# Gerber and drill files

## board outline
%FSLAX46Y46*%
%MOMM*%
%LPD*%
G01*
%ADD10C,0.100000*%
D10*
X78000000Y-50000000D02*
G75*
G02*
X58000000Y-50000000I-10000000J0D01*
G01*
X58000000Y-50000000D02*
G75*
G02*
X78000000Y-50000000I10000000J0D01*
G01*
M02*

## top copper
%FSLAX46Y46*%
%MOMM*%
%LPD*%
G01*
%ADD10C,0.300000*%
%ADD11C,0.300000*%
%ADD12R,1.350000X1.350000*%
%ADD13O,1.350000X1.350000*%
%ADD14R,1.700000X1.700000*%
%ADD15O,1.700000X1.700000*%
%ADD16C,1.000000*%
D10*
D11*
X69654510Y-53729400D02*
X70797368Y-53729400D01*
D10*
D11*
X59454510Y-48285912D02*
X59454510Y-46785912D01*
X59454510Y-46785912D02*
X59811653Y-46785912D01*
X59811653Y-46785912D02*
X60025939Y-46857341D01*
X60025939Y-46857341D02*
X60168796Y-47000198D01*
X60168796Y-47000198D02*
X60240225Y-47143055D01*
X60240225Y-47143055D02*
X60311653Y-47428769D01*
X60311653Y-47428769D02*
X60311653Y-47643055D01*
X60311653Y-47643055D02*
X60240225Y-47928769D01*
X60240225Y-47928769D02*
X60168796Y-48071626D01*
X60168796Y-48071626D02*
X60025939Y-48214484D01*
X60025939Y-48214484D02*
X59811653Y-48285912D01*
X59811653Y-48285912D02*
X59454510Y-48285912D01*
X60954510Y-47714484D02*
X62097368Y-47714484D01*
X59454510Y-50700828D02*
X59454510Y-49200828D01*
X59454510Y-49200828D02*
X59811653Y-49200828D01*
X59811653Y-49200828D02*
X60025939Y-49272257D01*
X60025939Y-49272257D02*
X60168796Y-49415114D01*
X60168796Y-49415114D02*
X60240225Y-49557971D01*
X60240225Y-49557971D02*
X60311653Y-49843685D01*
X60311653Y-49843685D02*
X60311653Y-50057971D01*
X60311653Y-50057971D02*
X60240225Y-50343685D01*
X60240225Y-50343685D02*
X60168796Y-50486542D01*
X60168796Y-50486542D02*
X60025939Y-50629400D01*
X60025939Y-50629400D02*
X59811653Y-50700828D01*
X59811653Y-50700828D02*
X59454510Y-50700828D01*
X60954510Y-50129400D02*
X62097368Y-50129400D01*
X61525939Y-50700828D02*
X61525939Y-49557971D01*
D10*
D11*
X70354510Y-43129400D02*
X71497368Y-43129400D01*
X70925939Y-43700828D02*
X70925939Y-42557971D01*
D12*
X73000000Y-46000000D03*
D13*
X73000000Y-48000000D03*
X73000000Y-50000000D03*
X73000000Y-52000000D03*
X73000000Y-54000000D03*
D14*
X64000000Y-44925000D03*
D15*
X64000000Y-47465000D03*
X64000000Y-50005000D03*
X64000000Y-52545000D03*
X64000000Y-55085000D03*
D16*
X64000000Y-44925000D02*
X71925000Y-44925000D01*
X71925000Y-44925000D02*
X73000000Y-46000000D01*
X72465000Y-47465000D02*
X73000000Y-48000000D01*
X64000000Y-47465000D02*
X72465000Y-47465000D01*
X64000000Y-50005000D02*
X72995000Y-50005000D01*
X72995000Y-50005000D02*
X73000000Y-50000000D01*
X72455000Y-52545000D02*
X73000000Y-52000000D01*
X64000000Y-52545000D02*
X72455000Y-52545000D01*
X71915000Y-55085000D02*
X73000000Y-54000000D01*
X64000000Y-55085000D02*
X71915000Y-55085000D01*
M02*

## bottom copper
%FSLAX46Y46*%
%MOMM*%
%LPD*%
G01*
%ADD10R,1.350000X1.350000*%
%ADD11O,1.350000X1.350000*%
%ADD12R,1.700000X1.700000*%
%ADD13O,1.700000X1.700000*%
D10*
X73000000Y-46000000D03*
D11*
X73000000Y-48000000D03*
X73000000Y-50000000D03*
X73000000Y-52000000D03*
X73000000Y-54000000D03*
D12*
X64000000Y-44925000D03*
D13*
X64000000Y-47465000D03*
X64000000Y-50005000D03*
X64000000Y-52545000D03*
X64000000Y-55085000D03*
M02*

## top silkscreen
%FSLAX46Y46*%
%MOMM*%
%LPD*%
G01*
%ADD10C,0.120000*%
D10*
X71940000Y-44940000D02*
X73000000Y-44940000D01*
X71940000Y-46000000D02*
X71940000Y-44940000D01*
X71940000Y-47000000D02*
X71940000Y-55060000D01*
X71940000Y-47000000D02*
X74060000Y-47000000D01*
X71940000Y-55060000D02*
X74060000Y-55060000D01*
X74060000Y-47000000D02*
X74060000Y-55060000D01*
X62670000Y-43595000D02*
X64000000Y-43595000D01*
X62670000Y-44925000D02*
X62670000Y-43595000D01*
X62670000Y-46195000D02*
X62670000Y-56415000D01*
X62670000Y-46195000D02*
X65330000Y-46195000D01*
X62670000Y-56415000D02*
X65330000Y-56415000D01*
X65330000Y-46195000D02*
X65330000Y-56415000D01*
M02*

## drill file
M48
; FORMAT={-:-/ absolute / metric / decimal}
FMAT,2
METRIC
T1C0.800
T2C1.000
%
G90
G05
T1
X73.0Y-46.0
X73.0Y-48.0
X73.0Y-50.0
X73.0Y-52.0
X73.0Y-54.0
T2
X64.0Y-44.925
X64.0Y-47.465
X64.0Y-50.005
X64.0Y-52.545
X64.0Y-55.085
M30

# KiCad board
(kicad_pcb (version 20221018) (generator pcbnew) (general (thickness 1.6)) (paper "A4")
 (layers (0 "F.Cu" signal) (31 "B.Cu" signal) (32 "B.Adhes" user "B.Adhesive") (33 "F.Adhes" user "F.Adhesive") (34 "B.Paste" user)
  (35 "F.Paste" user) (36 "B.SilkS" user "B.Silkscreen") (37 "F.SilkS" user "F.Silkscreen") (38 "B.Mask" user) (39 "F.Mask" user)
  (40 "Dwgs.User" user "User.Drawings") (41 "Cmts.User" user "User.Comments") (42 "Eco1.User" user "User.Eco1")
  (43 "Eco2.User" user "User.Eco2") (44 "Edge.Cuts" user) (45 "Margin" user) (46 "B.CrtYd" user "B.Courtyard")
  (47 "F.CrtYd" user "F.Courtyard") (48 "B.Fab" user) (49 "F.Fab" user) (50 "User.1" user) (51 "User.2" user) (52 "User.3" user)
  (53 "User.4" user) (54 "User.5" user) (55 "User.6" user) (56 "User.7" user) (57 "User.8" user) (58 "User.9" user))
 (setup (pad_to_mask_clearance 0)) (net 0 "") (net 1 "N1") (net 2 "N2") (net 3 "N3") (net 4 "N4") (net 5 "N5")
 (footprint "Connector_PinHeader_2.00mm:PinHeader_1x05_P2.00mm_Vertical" (layer "F.Cu") (at 73 46)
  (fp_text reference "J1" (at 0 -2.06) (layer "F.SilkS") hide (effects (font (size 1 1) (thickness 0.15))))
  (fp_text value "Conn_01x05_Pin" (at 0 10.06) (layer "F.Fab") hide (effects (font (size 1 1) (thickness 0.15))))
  (fp_line (start -1.06 -1.06) (end 0 -1.06) (stroke (width 0.12) (type solid)) (layer "F.SilkS"))
  (fp_line (start -1.06 0) (end -1.06 -1.06) (stroke (width 0.12) (type solid)) (layer "F.SilkS"))
  (fp_line (start -1.06 1) (end -1.06 9.06) (stroke (width 0.12) (type solid)) (layer "F.SilkS"))
  (fp_line (start -1.06 1) (end 1.06 1) (stroke (width 0.12) (type solid)) (layer "F.SilkS"))
  (fp_line (start -1.06 9.06) (end 1.06 9.06) (stroke (width 0.12) (type solid)) (layer "F.SilkS"))
  (fp_line (start 1.06 1) (end 1.06 9.06) (stroke (width 0.12) (type solid)) (layer "F.SilkS"))
  (pad "1" thru_hole rect (at 0 0) (size 1.35 1.35) (drill 0.8) (layers "*.Cu" "*.Mask") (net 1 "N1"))
  (pad "2" thru_hole oval (at 0 2) (size 1.35 1.35) (drill 0.8) (layers "*.Cu" "*.Mask") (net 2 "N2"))
  (pad "3" thru_hole oval (at 0 4) (size 1.35 1.35) (drill 0.8) (layers "*.Cu" "*.Mask") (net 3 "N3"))
  (pad "4" thru_hole oval (at 0 6) (size 1.35 1.35) (drill 0.8) (layers "*.Cu" "*.Mask") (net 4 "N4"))
  (pad "5" thru_hole oval (at 0 8) (size 1.35 1.35) (drill 0.8) (layers "*.Cu" "*.Mask") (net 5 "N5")))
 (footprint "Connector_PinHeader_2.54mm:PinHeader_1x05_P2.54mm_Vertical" (layer "F.Cu") (at 64 44.925)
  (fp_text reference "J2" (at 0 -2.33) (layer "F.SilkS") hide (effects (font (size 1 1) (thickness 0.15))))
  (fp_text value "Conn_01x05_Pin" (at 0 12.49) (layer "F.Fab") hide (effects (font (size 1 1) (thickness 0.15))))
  (fp_line (start -1.33 -1.33) (end 0 -1.33) (stroke (width 0.12) (type solid)) (layer "F.SilkS"))
  (fp_line (start -1.33 0) (end -1.33 -1.33) (stroke (width 0.12) (type solid)) (layer "F.SilkS"))
  (fp_line (start -1.33 1.27) (end -1.33 11.49) (stroke (width 0.12) (type solid)) (layer "F.SilkS"))
  (fp_line (start -1.33 1.27) (end 1.33 1.27) (stroke (width 0.12) (type solid)) (layer "F.SilkS"))
  (fp_line (start -1.33 11.49) (end 1.33 11.49) (stroke (width 0.12) (type solid)) (layer "F.SilkS"))
  (fp_line (start 1.33 1.27) (end 1.33 11.49) (stroke (width 0.12) (type solid)) (layer "F.SilkS"))
  (pad "1" thru_hole rect (at 0 0) (size 1.7 1.7) (drill 1) (layers "*.Cu" "*.Mask") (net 1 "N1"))
  (pad "2" thru_hole oval (at 0 2.54) (size 1.7 1.7) (drill 1) (layers "*.Cu" "*.Mask") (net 2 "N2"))
  (pad "3" thru_hole oval (at 0 5.08) (size 1.7 1.7) (drill 1) (layers "*.Cu" "*.Mask") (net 3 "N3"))
  (pad "4" thru_hole oval (at 0 7.62) (size 1.7 1.7) (drill 1) (layers "*.Cu" "*.Mask") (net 4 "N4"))
  (pad "5" thru_hole oval (at 0 10.16) (size 1.7 1.7) (drill 1) (layers "*.Cu" "*.Mask") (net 5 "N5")))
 (gr_circle (center 68 50) (end 78 50) (stroke (width 0.1) (type default)) (fill none) (layer "Edge.Cuts"))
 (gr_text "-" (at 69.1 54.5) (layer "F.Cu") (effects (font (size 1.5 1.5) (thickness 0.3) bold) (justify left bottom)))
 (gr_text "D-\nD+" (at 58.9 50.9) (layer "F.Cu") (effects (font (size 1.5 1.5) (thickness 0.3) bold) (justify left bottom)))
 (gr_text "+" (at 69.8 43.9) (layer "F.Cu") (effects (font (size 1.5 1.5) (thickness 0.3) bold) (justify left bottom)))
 (segment (start 64 44.925) (end 71.925 44.925) (width 1) (layer "F.Cu") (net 1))
 (segment (start 71.925 44.925) (end 73 46) (width 1) (layer "F.Cu") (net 1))
 (segment (start 72.465 47.465) (end 73 48) (width 1) (layer "F.Cu") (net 2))
 (segment (start 64 47.465) (end 72.465 47.465) (width 1) (layer "F.Cu") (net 2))
 (segment (start 64 50.005) (end 72.995 50.005) (width 1) (layer "F.Cu") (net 3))
 (segment (start 72.995 50.005) (end 73 50) (width 1) (layer "F.Cu") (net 3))
 (segment (start 72.455 52.545) (end 73 52) (width 1) (layer "F.Cu") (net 4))
 (segment (start 64 52.545) (end 72.455 52.545) (width 1) (layer "F.Cu") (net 4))
 (segment (start 71.915 55.085) (end 73 54) (width 1) (layer "F.Cu") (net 5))
 (segment (start 64 55.085) (end 71.915 55.085) (width 1) (layer "F.Cu") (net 5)))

